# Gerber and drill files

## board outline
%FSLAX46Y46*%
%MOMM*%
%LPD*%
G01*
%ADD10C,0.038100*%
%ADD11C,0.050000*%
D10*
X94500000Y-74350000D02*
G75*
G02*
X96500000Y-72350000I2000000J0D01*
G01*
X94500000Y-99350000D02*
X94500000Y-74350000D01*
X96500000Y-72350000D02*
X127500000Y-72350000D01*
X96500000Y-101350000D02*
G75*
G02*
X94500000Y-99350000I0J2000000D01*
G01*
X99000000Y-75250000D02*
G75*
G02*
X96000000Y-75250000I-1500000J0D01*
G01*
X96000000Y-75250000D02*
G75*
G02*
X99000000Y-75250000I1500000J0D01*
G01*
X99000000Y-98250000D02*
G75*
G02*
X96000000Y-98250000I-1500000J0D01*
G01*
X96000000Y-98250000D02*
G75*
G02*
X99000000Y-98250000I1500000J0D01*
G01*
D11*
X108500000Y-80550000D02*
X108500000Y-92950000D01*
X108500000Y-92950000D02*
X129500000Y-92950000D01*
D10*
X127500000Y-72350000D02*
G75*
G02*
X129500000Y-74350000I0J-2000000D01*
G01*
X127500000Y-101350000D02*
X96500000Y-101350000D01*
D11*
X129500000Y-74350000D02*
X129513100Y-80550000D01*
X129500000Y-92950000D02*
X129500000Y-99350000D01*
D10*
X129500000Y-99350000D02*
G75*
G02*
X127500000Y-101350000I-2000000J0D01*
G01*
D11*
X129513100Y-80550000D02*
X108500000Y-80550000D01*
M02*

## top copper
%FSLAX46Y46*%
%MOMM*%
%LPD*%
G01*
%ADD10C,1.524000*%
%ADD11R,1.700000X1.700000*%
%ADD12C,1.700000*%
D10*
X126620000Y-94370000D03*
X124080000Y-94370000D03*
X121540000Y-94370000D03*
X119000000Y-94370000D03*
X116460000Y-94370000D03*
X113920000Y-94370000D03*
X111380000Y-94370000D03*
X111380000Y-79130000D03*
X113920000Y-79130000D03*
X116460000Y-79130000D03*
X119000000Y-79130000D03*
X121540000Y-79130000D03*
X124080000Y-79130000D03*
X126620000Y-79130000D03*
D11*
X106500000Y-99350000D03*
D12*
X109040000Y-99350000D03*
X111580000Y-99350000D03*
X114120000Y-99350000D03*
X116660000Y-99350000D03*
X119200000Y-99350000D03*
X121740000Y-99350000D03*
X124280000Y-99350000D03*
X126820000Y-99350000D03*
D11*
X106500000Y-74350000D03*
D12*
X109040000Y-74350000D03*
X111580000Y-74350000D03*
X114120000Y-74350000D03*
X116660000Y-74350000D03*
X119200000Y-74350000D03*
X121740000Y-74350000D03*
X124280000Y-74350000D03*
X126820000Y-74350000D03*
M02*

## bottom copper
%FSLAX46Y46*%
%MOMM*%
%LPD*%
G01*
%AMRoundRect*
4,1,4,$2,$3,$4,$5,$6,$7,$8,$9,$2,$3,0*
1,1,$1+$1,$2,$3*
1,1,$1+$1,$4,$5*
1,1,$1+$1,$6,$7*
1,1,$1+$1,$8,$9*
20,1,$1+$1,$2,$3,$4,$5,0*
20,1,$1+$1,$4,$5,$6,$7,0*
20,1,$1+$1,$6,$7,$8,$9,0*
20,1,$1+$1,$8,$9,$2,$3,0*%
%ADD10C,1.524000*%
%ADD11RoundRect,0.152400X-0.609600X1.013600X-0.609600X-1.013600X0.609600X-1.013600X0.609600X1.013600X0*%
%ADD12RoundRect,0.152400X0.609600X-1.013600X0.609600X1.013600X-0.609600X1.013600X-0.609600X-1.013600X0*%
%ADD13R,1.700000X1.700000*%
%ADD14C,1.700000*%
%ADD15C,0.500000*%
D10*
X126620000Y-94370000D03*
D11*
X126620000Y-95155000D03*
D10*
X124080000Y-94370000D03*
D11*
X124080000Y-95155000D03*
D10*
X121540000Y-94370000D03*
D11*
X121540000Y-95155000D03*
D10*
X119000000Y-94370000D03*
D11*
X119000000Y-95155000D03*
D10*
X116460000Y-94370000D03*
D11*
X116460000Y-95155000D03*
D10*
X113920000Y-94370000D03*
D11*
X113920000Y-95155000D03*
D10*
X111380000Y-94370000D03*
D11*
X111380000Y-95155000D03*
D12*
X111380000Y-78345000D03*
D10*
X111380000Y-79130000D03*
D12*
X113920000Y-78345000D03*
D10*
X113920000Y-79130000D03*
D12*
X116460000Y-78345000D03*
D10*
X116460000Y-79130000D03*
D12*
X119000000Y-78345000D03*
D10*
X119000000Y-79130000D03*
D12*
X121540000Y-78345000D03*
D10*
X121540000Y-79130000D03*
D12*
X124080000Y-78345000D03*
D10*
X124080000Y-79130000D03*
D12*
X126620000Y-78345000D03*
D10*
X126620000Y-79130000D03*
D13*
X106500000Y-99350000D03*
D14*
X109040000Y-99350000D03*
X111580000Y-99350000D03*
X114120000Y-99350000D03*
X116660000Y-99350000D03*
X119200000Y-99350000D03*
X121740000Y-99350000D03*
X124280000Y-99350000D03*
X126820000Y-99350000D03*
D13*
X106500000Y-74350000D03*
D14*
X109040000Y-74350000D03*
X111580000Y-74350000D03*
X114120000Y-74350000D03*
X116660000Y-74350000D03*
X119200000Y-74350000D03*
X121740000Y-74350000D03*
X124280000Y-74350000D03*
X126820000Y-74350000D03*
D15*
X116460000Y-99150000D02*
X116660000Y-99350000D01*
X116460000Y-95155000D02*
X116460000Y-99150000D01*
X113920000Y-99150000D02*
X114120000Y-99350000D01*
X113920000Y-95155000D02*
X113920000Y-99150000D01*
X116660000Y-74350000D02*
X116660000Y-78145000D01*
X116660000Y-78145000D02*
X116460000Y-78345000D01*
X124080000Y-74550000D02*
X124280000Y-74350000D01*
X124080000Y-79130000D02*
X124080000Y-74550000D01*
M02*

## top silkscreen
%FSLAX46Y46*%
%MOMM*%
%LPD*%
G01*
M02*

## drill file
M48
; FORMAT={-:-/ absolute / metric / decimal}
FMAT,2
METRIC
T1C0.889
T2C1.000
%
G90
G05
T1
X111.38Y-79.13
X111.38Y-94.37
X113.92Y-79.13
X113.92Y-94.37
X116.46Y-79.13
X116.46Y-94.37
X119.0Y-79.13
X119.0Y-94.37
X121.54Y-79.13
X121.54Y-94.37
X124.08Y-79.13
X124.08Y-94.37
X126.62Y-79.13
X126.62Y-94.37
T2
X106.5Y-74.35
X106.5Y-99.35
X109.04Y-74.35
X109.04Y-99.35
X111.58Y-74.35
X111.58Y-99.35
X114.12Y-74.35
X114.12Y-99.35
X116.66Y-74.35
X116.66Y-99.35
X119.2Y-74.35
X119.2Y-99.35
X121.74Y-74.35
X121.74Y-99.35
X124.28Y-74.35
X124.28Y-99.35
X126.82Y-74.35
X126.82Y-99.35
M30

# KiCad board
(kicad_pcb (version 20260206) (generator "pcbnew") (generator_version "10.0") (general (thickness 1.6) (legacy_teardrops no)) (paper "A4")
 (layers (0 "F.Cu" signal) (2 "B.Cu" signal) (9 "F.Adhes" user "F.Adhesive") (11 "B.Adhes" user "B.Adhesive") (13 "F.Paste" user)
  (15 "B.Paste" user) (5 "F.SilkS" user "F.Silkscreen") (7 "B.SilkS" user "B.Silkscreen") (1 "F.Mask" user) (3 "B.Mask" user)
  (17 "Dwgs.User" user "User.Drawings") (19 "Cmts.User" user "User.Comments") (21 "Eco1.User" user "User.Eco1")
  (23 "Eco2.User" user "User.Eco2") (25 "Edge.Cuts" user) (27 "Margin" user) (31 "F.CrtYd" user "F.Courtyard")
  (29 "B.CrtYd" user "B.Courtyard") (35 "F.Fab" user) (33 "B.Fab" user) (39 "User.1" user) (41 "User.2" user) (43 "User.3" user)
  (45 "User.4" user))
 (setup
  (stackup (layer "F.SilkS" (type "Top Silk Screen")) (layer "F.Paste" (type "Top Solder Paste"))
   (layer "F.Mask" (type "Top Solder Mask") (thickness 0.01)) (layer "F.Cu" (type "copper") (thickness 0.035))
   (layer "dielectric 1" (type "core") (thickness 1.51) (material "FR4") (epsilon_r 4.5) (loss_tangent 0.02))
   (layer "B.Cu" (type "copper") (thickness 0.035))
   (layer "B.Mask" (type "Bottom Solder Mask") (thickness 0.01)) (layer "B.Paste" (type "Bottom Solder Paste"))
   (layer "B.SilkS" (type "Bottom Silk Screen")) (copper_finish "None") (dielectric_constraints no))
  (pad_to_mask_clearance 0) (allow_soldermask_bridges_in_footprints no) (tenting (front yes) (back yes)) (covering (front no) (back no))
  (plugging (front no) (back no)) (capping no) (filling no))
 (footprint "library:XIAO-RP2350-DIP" (layer "B.Cu") (at 119 86.75)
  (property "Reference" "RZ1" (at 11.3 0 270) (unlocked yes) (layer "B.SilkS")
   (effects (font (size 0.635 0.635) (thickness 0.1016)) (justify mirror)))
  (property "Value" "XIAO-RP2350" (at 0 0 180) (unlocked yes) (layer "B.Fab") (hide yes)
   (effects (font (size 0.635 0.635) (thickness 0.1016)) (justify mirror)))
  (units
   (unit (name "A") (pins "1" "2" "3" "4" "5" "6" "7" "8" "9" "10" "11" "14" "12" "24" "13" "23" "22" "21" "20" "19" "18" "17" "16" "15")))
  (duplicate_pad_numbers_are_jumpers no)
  (pad "1" thru_hole circle (at 7.62 7.62 270) (size 1.524 1.524) (drill 0.889) (layers "*.Cu" "*.Mask") (remove_unused_layers no)
   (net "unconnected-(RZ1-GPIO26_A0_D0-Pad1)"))
  (pad "1" smd roundrect (at 7.62 8.405 270) (size 2.332 1.524) (layers "B.Cu" "B.Mask") (roundrect_rratio 0.1)
   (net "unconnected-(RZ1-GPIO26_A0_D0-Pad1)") (thermal_bridge_angle 45))
  (pad "2" thru_hole circle (at 5.08 7.62 270) (size 1.524 1.524) (drill 0.889) (layers "*.Cu" "*.Mask") (remove_unused_layers no)
   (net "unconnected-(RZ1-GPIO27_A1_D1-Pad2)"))
  (pad "2" smd roundrect (at 5.08 8.405 270) (size 2.332 1.524) (layers "B.Cu" "B.Mask") (roundrect_rratio 0.1)
   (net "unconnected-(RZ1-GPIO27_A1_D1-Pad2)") (thermal_bridge_angle 45))
  (pad "3" thru_hole circle (at 2.54 7.62 270) (size 1.524 1.524) (drill 0.889) (layers "*.Cu" "*.Mask") (remove_unused_layers no)
   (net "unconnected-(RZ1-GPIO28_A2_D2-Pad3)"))
  (pad "3" smd roundrect (at 2.54 8.405 270) (size 2.332 1.524) (layers "B.Cu" "B.Mask") (roundrect_rratio 0.1)
   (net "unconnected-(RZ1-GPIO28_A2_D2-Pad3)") (thermal_bridge_angle 45))
  (pad "4" thru_hole circle (at 0 7.62 270) (size 1.524 1.524) (drill 0.889) (layers "*.Cu" "*.Mask") (remove_unused_layers no)
   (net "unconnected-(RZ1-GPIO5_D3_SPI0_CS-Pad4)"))
  (pad "4" smd roundrect (at 0 8.405 270) (size 2.332 1.524) (layers "B.Cu" "B.Mask") (roundrect_rratio 0.1)
   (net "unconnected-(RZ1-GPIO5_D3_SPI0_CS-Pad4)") (thermal_bridge_angle 45))
  (pad "5" thru_hole circle (at -2.54 7.62 270) (size 1.524 1.524) (drill 0.889) (layers "*.Cu" "*.Mask") (remove_unused_layers no)
   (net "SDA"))
  (pad "5" smd roundrect (at -2.54 8.405 270) (size 2.332 1.524) (layers "B.Cu" "B.Mask") (roundrect_rratio 0.1) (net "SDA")
   (thermal_bridge_angle 45))
  (pad "6" thru_hole circle (at -5.08 7.62 270) (size 1.524 1.524) (drill 0.889) (layers "*.Cu" "*.Mask") (remove_unused_layers no)
   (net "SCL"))
  (pad "6" smd roundrect (at -5.08 8.405 270) (size 2.332 1.524) (layers "B.Cu" "B.Mask") (roundrect_rratio 0.1) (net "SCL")
   (thermal_bridge_angle 45))
  (pad "7" thru_hole circle (at -7.62 7.62 270) (size 1.524 1.524) (drill 0.889) (layers "*.Cu" "*.Mask") (remove_unused_layers no)
   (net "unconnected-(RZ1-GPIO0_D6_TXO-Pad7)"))
  (pad "7" smd roundrect (at -7.62 8.405 270) (size 2.332 1.524) (layers "B.Cu" "B.Mask") (roundrect_rratio 0.1)
   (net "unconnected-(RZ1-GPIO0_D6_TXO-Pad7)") (thermal_bridge_angle 45))
  (pad "8" smd roundrect (at -7.62 -8.405 90) (size 2.332 1.524) (layers "B.Cu" "B.Mask") (roundrect_rratio 0.1)
   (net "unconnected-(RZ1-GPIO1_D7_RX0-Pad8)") (thermal_bridge_angle 45))
  (pad "8" thru_hole circle (at -7.62 -7.62 90) (size 1.524 1.524) (drill 0.889) (layers "*.Cu" "*.Mask") (remove_unused_layers no)
   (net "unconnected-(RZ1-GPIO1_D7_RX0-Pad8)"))
  (pad "9" smd roundrect (at -5.08 -8.405 90) (size 2.332 1.524) (layers "B.Cu" "B.Mask") (roundrect_rratio 0.1)
   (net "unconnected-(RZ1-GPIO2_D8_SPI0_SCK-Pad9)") (thermal_bridge_angle 45))
  (pad "9" thru_hole circle (at -5.08 -7.62 90) (size 1.524 1.524) (drill 0.889) (layers "*.Cu" "*.Mask") (remove_unused_layers no)
   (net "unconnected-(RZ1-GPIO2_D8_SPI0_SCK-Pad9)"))
  (pad "10" smd roundrect (at -2.54 -8.405 90) (size 2.332 1.524) (layers "B.Cu" "B.Mask") (roundrect_rratio 0.1) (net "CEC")
   (thermal_bridge_angle 45))
  (pad "10" thru_hole circle (at -2.54 -7.62 90) (size 1.524 1.524) (drill 0.889) (layers "*.Cu" "*.Mask") (remove_unused_layers no)
   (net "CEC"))
  (pad "11" smd roundrect (at 0 -8.405 90) (size 2.332 1.524) (layers "B.Cu" "B.Mask") (roundrect_rratio 0.1)
   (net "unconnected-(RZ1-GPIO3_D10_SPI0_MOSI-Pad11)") (thermal_bridge_angle 45))
  (pad "11" thru_hole circle (at 0 -7.62 90) (size 1.524 1.524) (drill 0.889) (layers "*.Cu" "*.Mask") (remove_unused_layers no)
   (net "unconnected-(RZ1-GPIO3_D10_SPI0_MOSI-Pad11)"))
  (pad "12" smd roundrect (at 2.54 -8.405 90) (size 2.332 1.524) (layers "B.Cu" "B.Mask") (roundrect_rratio 0.1)
   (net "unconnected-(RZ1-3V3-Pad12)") (thermal_bridge_angle 45))
  (pad "12" thru_hole circle (at 2.54 -7.62 90) (size 1.524 1.524) (drill 0.889) (layers "*.Cu" "*.Mask") (remove_unused_layers no)
   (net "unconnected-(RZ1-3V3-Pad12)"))
  (pad "13" smd roundrect (at 5.08 -8.405 90) (size 2.332 1.524) (layers "B.Cu" "B.Mask") (roundrect_rratio 0.1) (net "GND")
   (thermal_bridge_angle 45))
  (pad "13" thru_hole circle (at 5.08 -7.62 90) (size 1.524 1.524) (drill 0.889) (layers "*.Cu" "*.Mask") (remove_unused_layers no)
   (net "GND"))
  (pad "14" smd roundrect (at 7.62 -8.405 90) (size 2.332 1.524) (layers "B.Cu" "B.Mask") (roundrect_rratio 0.1)
   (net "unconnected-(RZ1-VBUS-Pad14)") (thermal_bridge_angle 45))
  (pad "14" thru_hole circle (at 7.62 -7.62 90) (size 1.524 1.524) (drill 0.889) (layers "*.Cu" "*.Mask") (remove_unused_layers no)
   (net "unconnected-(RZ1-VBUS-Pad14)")))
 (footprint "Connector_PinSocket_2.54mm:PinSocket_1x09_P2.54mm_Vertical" (layer "B.Cu") (at 106.5 99.35 -90)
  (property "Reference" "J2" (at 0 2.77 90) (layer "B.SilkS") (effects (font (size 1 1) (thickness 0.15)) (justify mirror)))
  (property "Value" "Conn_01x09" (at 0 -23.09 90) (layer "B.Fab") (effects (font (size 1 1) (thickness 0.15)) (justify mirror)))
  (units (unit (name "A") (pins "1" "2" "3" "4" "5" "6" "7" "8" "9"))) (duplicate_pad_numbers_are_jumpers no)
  (pad "1" thru_hole rect (at 0 0 270) (size 1.7 1.7) (drill 1) (layers "*.Cu" "*.Mask") (remove_unused_layers no)
   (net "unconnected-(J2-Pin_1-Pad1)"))
  (pad "2" thru_hole circle (at 0 -2.54 270) (size 1.7 1.7) (drill 1) (layers "*.Cu" "*.Mask") (remove_unused_layers no)
   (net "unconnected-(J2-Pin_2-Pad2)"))
  (pad "3" thru_hole circle (at 0 -5.08 270) (size 1.7 1.7) (drill 1) (layers "*.Cu" "*.Mask") (remove_unused_layers no)
   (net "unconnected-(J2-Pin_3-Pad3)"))
  (pad "4" thru_hole circle (at 0 -7.62 270) (size 1.7 1.7) (drill 1) (layers "*.Cu" "*.Mask") (remove_unused_layers no) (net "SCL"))
  (pad "5" thru_hole circle (at 0 -10.16 270) (size 1.7 1.7) (drill 1) (layers "*.Cu" "*.Mask") (remove_unused_layers no) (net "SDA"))
  (pad "6" thru_hole circle (at 0 -12.7 270) (size 1.7 1.7) (drill 1) (layers "*.Cu" "*.Mask") (remove_unused_layers no)
   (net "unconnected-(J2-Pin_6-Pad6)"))
  (pad "7" thru_hole circle (at 0 -15.24 270) (size 1.7 1.7) (drill 1) (layers "*.Cu" "*.Mask") (remove_unused_layers no)
   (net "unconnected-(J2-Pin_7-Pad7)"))
  (pad "8" thru_hole circle (at 0 -17.78 270) (size 1.7 1.7) (drill 1) (layers "*.Cu" "*.Mask") (remove_unused_layers no)
   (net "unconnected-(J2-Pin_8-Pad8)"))
  (pad "9" thru_hole circle (at 0 -20.32 270) (size 1.7 1.7) (drill 1) (layers "*.Cu" "*.Mask") (remove_unused_layers no)
   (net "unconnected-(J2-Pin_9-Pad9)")))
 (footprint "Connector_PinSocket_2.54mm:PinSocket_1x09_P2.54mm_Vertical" (layer "B.Cu") (at 106.5 74.35 -90)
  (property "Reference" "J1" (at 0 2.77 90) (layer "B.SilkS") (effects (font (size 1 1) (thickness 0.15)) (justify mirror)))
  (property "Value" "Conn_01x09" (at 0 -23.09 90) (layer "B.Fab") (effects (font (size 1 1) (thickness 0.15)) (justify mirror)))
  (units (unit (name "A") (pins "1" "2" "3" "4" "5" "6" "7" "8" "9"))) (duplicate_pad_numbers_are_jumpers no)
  (pad "1" thru_hole rect (at 0 0 270) (size 1.7 1.7) (drill 1) (layers "*.Cu" "*.Mask") (remove_unused_layers no)
   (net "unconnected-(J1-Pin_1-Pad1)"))
  (pad "2" thru_hole circle (at 0 -2.54 270) (size 1.7 1.7) (drill 1) (layers "*.Cu" "*.Mask") (remove_unused_layers no)
   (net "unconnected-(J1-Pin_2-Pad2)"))
  (pad "3" thru_hole circle (at 0 -5.08 270) (size 1.7 1.7) (drill 1) (layers "*.Cu" "*.Mask") (remove_unused_layers no)
   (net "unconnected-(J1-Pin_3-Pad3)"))
  (pad "4" thru_hole circle (at 0 -7.62 270) (size 1.7 1.7) (drill 1) (layers "*.Cu" "*.Mask") (remove_unused_layers no)
   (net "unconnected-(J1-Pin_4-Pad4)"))
  (pad "5" thru_hole circle (at 0 -10.16 270) (size 1.7 1.7) (drill 1) (layers "*.Cu" "*.Mask") (remove_unused_layers no) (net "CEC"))
  (pad "6" thru_hole circle (at 0 -12.7 270) (size 1.7 1.7) (drill 1) (layers "*.Cu" "*.Mask") (remove_unused_layers no)
   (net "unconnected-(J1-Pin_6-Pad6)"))
  (pad "7" thru_hole circle (at 0 -15.24 270) (size 1.7 1.7) (drill 1) (layers "*.Cu" "*.Mask") (remove_unused_layers no)
   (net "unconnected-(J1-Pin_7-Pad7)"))
  (pad "8" thru_hole circle (at 0 -17.78 270) (size 1.7 1.7) (drill 1) (layers "*.Cu" "*.Mask") (remove_unused_layers no) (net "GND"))
  (pad "9" thru_hole circle (at 0 -20.32 270) (size 1.7 1.7) (drill 1) (layers "*.Cu" "*.Mask") (remove_unused_layers no)
   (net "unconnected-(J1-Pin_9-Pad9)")))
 (gr_arc (start 94.5 74.35) (mid 95.085786 72.935786) (end 96.5 72.35) (stroke (width 0.0381) (type default)) (layer "Edge.Cuts"))
 (gr_line (start 94.5 99.35) (end 94.5 74.35) (stroke (width 0.0381) (type default)) (layer "Edge.Cuts"))
 (gr_line (start 96.5 72.35) (end 127.5 72.35) (stroke (width 0.0381) (type default)) (layer "Edge.Cuts"))
 (gr_arc (start 96.5 101.35) (mid 95.085786 100.764214) (end 94.5 99.35) (stroke (width 0.0381) (type default)) (layer "Edge.Cuts"))
 (gr_circle (center 97.5 75.25) (end 99 75.25) (stroke (width 0.0381) (type default)) (fill no) (layer "Edge.Cuts"))
 (gr_circle (center 97.5 98.25) (end 99 98.25) (stroke (width 0.0381) (type default)) (fill no) (layer "Edge.Cuts"))
 (gr_line (start 108.5 80.55) (end 108.5 92.95) (stroke (width 0.05) (type default)) (layer "Edge.Cuts"))
 (gr_line (start 108.5 92.95) (end 129.5 92.95) (stroke (width 0.05) (type default)) (layer "Edge.Cuts"))
 (gr_arc (start 127.5 72.35) (mid 128.914214 72.935786) (end 129.5 74.35) (stroke (width 0.0381) (type default)) (layer "Edge.Cuts"))
 (gr_line (start 127.5 101.35) (end 96.5 101.35) (stroke (width 0.0381) (type default)) (layer "Edge.Cuts"))
 (gr_line (start 129.5 74.35) (end 129.5131 80.55) (stroke (width 0.05) (type default)) (layer "Edge.Cuts"))
 (gr_line (start 129.5 92.95) (end 129.5 99.35) (stroke (width 0.05) (type default)) (layer "Edge.Cuts"))
 (gr_arc (start 129.5 99.35) (mid 128.914214 100.764214) (end 127.5 101.35) (stroke (width 0.0381) (type default)) (layer "Edge.Cuts"))
 (gr_line (start 129.5131 80.55) (end 108.5 80.55) (stroke (width 0.05) (type default)) (layer "Edge.Cuts"))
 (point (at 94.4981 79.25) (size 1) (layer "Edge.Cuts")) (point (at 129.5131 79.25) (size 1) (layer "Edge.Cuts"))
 (segment (start 116.46 99.15) (end 116.66 99.35) (width 0.5) (layer "B.Cu") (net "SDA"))
 (segment (start 116.46 95.155) (end 116.46 99.15) (width 0.5) (layer "B.Cu") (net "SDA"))
 (segment (start 113.92 99.15) (end 114.12 99.35) (width 0.5) (layer "B.Cu") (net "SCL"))
 (segment (start 113.92 95.155) (end 113.92 99.15) (width 0.5) (layer "B.Cu") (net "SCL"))
 (segment (start 116.66 74.35) (end 116.66 78.145) (width 0.5) (layer "B.Cu") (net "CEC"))
 (segment (start 116.66 78.145) (end 116.46 78.345) (width 0.5) (layer "B.Cu") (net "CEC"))
 (segment (start 124.08 74.55) (end 124.28 74.35) (width 0.5) (layer "B.Cu") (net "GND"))
 (segment (start 124.08 79.13) (end 124.08 74.55) (width 0.5) (layer "B.Cu") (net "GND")))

